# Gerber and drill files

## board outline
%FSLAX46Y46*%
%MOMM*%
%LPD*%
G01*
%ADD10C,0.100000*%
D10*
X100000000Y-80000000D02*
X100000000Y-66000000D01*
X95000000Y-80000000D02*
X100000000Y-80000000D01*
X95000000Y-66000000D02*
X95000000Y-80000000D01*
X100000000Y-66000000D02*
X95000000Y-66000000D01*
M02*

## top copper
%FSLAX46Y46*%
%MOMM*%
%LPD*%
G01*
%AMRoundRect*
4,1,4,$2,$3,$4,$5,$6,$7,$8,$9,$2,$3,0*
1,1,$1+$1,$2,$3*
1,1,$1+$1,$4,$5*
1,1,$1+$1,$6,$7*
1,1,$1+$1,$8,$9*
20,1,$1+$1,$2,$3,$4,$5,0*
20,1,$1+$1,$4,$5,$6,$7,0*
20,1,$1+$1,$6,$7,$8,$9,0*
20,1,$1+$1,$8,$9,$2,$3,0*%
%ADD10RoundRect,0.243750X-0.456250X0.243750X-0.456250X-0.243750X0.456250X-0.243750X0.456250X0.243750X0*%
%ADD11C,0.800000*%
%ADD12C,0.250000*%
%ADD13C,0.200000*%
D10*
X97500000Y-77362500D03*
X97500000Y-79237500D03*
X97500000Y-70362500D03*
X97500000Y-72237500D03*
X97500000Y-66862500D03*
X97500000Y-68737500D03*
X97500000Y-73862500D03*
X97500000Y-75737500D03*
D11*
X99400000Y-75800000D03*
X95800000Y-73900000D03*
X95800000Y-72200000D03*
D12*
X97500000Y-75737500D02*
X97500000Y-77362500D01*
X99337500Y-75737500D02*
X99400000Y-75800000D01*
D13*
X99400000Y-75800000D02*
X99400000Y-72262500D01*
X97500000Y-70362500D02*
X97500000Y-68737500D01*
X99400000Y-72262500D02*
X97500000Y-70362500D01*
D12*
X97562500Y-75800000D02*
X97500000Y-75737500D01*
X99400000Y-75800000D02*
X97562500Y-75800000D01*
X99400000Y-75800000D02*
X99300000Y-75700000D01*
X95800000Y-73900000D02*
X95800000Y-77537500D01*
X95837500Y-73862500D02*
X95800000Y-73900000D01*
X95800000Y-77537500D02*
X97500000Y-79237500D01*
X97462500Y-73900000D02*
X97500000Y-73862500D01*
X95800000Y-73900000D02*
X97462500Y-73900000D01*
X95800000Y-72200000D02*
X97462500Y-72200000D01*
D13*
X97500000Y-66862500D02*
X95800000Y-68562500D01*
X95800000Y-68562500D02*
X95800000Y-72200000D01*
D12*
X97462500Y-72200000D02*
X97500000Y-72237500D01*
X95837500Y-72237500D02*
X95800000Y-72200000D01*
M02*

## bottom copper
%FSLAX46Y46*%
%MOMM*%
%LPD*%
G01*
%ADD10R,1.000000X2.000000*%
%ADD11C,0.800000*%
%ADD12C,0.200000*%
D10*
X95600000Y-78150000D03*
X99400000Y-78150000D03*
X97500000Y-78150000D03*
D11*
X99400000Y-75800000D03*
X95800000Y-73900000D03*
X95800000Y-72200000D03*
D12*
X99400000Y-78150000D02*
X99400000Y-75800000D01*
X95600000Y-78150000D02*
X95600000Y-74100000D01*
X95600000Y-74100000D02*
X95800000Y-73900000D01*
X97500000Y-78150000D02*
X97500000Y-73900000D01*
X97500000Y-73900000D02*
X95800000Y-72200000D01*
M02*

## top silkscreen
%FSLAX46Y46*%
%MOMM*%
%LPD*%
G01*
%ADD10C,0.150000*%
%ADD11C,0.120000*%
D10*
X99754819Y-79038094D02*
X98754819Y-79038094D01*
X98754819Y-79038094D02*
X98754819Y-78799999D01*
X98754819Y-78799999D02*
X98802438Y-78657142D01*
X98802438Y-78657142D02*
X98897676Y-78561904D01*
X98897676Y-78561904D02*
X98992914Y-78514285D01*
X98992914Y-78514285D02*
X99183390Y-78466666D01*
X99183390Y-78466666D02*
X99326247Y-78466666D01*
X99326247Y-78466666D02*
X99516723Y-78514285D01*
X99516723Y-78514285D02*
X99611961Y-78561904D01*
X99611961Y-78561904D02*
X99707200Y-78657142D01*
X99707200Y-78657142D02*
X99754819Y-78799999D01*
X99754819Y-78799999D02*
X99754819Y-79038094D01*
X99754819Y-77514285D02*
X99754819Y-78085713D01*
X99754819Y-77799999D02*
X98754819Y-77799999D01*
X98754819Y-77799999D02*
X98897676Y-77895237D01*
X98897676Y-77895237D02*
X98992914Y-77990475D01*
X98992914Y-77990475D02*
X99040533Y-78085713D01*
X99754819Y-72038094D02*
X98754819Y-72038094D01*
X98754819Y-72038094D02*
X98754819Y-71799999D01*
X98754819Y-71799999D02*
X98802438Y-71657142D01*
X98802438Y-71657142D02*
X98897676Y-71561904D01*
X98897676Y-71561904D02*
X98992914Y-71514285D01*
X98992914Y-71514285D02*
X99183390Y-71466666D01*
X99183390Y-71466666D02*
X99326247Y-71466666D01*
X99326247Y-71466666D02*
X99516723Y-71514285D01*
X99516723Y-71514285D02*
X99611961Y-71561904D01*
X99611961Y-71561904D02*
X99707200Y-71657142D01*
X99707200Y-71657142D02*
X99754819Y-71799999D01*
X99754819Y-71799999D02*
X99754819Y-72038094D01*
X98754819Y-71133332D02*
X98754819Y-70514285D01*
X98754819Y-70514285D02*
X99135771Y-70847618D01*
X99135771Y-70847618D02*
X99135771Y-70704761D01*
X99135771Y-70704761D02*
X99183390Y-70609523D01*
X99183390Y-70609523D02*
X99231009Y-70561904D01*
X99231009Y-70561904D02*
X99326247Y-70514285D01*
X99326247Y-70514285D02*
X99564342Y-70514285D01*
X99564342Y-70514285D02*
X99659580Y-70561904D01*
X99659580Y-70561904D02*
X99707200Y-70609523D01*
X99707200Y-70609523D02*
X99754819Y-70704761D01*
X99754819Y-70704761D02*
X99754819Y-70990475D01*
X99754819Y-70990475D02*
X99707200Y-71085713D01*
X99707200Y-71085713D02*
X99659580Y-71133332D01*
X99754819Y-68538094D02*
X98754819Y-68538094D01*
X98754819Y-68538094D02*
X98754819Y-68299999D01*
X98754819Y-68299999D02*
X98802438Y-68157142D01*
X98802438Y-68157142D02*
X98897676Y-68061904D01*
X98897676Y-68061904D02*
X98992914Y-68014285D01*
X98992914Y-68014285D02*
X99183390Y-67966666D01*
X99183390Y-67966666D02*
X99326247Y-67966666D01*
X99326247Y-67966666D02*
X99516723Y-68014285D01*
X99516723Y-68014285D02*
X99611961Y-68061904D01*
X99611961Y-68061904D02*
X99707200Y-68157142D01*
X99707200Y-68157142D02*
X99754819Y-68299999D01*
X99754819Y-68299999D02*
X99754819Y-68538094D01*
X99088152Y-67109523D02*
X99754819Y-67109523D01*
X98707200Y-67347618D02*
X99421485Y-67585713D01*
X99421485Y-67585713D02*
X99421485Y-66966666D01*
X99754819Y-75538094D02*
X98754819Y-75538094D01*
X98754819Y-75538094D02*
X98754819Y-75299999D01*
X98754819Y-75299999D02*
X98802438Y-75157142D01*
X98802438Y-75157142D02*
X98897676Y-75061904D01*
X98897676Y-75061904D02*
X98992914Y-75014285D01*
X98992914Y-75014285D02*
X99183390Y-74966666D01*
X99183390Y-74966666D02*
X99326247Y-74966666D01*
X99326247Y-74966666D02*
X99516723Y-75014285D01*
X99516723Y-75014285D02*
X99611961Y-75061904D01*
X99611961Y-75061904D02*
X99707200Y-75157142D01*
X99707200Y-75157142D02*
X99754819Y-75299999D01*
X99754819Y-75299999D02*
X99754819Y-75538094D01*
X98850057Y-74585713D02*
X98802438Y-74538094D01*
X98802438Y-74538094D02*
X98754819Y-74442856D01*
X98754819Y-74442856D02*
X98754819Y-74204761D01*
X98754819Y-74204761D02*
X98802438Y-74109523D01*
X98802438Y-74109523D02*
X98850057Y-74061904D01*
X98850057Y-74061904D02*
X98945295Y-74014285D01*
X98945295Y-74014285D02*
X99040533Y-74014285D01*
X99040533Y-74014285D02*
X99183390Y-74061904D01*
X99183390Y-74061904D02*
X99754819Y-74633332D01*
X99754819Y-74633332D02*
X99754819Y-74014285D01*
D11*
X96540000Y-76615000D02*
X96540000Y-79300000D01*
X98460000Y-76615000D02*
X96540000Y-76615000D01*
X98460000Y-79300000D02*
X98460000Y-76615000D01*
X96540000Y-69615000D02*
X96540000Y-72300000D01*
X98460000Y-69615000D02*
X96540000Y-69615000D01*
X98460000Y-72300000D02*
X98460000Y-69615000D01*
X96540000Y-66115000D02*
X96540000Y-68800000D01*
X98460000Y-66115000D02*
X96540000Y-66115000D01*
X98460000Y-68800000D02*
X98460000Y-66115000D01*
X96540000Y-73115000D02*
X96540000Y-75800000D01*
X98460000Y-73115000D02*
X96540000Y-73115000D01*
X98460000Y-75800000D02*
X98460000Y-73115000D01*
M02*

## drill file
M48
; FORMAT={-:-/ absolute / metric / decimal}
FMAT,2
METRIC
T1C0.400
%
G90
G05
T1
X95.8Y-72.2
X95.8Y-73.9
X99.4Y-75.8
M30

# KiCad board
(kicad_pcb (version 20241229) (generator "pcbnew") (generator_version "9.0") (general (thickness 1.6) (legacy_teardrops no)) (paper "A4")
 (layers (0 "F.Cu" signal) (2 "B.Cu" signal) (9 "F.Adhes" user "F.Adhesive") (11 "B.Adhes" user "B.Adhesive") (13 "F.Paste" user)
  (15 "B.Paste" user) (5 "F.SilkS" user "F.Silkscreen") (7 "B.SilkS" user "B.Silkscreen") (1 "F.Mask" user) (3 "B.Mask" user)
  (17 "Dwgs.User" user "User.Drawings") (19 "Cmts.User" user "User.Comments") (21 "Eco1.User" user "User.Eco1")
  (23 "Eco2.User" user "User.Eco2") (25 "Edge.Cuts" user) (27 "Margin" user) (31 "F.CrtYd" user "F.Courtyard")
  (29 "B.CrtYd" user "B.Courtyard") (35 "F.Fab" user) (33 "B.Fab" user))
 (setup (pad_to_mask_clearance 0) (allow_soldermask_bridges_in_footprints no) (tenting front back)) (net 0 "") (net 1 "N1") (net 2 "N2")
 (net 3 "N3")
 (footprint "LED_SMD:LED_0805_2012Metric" (layer "F.Cu") (at 97.5 78.3 -90)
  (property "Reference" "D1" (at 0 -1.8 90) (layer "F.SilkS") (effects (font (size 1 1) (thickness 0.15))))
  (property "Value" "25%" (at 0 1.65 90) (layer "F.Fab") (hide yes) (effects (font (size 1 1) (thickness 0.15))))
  (fp_line (start -1.685 0.96) (end 1 0.96) (stroke (width 0.12) (type solid)) (layer "F.SilkS"))
  (fp_line (start -1.685 -0.96) (end -1.685 0.96) (stroke (width 0.12) (type solid)) (layer "F.SilkS"))
  (fp_line (start 1 -0.96) (end -1.685 -0.96) (stroke (width 0.12) (type solid)) (layer "F.SilkS"))
  (pad "1" smd roundrect (at -0.9375 0 270) (size 0.975 1.4) (layers "F.Cu" "F.Mask" "F.Paste") (roundrect_rratio 0.25) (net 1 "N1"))
  (pad "2" smd roundrect (at 0.9375 0 270) (size 0.975 1.4) (layers "F.Cu" "F.Mask" "F.Paste") (roundrect_rratio 0.25) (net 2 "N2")))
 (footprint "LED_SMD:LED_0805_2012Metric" (layer "F.Cu") (at 97.5 71.3 -90)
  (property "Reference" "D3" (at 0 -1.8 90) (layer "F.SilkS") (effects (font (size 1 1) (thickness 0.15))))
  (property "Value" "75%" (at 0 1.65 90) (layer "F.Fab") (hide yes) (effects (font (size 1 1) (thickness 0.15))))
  (fp_line (start -1.685 0.96) (end 1 0.96) (stroke (width 0.12) (type solid)) (layer "F.SilkS"))
  (fp_line (start -1.685 -0.96) (end -1.685 0.96) (stroke (width 0.12) (type solid)) (layer "F.SilkS"))
  (fp_line (start 1 -0.96) (end -1.685 -0.96) (stroke (width 0.12) (type solid)) (layer "F.SilkS"))
  (pad "1" smd roundrect (at -0.9375 0 270) (size 0.975 1.4) (layers "F.Cu" "F.Mask" "F.Paste") (roundrect_rratio 0.25) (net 1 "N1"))
  (pad "2" smd roundrect (at 0.9375 0 270) (size 0.975 1.4) (layers "F.Cu" "F.Mask" "F.Paste") (roundrect_rratio 0.25) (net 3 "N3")))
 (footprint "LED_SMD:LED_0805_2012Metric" (layer "F.Cu") (at 97.5 67.8 -90)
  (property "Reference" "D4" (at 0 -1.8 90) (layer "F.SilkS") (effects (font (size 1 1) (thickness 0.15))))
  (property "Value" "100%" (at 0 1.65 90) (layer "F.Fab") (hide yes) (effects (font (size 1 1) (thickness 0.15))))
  (fp_line (start -1.685 0.96) (end 1 0.96) (stroke (width 0.12) (type solid)) (layer "F.SilkS"))
  (fp_line (start -1.685 -0.96) (end -1.685 0.96) (stroke (width 0.12) (type solid)) (layer "F.SilkS"))
  (fp_line (start 1 -0.96) (end -1.685 -0.96) (stroke (width 0.12) (type solid)) (layer "F.SilkS"))
  (pad "1" smd roundrect (at -0.9375 0 270) (size 0.975 1.4) (layers "F.Cu" "F.Mask" "F.Paste") (roundrect_rratio 0.25) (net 3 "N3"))
  (pad "2" smd roundrect (at 0.9375 0 270) (size 0.975 1.4) (layers "F.Cu" "F.Mask" "F.Paste") (roundrect_rratio 0.25) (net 1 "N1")))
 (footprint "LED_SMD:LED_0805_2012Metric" (layer "F.Cu") (at 97.5 74.8 -90)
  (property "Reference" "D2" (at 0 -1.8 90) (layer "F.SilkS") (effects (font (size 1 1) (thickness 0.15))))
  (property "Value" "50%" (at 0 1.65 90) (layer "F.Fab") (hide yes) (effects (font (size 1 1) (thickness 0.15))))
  (fp_line (start -1.685 0.96) (end 1 0.96) (stroke (width 0.12) (type solid)) (layer "F.SilkS"))
  (fp_line (start -1.685 -0.96) (end -1.685 0.96) (stroke (width 0.12) (type solid)) (layer "F.SilkS"))
  (fp_line (start 1 -0.96) (end -1.685 -0.96) (stroke (width 0.12) (type solid)) (layer "F.SilkS"))
  (pad "1" smd roundrect (at -0.9375 0 270) (size 0.975 1.4) (layers "F.Cu" "F.Mask" "F.Paste") (roundrect_rratio 0.25) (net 2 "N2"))
  (pad "2" smd roundrect (at 0.9375 0 270) (size 0.975 1.4) (layers "F.Cu" "F.Mask" "F.Paste") (roundrect_rratio 0.25) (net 1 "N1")))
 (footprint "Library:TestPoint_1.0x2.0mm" (layer "B.Cu") (at 95.6 78.15 180)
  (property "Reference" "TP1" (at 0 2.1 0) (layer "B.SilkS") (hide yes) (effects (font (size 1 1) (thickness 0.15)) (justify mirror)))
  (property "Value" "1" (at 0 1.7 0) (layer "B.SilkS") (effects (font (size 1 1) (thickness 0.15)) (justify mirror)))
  (pad "1" smd rect (at 0 0 180) (size 1 2) (layers "B.Cu" "B.Mask") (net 2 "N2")))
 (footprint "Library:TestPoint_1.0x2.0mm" (layer "B.Cu") (at 99.4 78.15 180)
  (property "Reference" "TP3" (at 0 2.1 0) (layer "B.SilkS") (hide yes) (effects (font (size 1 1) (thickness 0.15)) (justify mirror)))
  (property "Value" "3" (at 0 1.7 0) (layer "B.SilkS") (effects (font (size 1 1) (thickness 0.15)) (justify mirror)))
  (pad "3" smd rect (at 0 0 180) (size 1 2) (layers "B.Cu" "B.Mask") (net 1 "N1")))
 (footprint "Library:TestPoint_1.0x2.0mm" (layer "B.Cu") (at 97.5 78.15 180)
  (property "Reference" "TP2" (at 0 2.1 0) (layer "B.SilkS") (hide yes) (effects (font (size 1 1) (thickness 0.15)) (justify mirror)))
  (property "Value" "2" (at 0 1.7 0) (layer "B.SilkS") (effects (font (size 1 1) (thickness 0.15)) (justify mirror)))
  (pad "2" smd rect (at 0 0 180) (size 1 2) (layers "B.Cu" "B.Mask") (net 3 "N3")))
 (gr_line (start 100 80) (end 100 66) (stroke (width 0.1) (type solid)) (layer "Edge.Cuts"))
 (gr_line (start 95 80) (end 100 80) (stroke (width 0.1) (type solid)) (layer "Edge.Cuts"))
 (gr_line (start 95 66) (end 95 80) (stroke (width 0.1) (type solid)) (layer "Edge.Cuts"))
 (gr_line (start 100 66) (end 95 66) (stroke (width 0.1) (type solid)) (layer "Edge.Cuts"))
 (segment (start 97.5 75.7375) (end 97.5 77.3625) (width 0.25) (layer "F.Cu") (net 1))
 (segment (start 99.3375 75.7375) (end 99.4 75.8) (width 0.25) (layer "F.Cu") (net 1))
 (segment (start 99.4 75.8) (end 99.4 72.2625) (width 0.2) (layer "F.Cu") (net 1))
 (segment (start 97.5 70.3625) (end 97.5 68.7375) (width 0.2) (layer "F.Cu") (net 1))
 (segment (start 99.4 72.2625) (end 97.5 70.3625) (width 0.2) (layer "F.Cu") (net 1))
 (segment (start 97.5625 75.8) (end 97.5 75.7375) (width 0.25) (layer "F.Cu") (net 1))
 (segment (start 99.4 75.8) (end 97.5625 75.8) (width 0.25) (layer "F.Cu") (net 1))
 (segment (start 99.4 75.8) (end 99.3 75.7) (width 0.25) (layer "F.Cu") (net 1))
 (via (at 99.4 75.8) (size 0.8) (drill 0.4) (layers "F.Cu" "B.Cu") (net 1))
 (segment (start 99.4 78.15) (end 99.4 75.8) (width 0.2) (layer "B.Cu") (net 1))
 (segment (start 95.8 73.9) (end 95.8 77.5375) (width 0.25) (layer "F.Cu") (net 2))
 (segment (start 95.8375 73.8625) (end 95.8 73.9) (width 0.25) (layer "F.Cu") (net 2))
 (segment (start 95.8 77.5375) (end 97.5 79.2375) (width 0.25) (layer "F.Cu") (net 2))
 (segment (start 97.4625 73.9) (end 97.5 73.8625) (width 0.25) (layer "F.Cu") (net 2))
 (segment (start 95.8 73.9) (end 97.4625 73.9) (width 0.25) (layer "F.Cu") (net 2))
 (via (at 95.8 73.9) (size 0.8) (drill 0.4) (layers "F.Cu" "B.Cu") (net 2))
 (segment (start 95.6 78.15) (end 95.6 74.1) (width 0.2) (layer "B.Cu") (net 2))
 (segment (start 95.6 74.1) (end 95.8 73.9) (width 0.2) (layer "B.Cu") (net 2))
 (segment (start 95.8 72.2) (end 97.4625 72.2) (width 0.25) (layer "F.Cu") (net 3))
 (segment (start 97.5 66.8625) (end 95.8 68.5625) (width 0.2) (layer "F.Cu") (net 3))
 (segment (start 95.8 68.5625) (end 95.8 72.2) (width 0.2) (layer "F.Cu") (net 3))
 (segment (start 97.4625 72.2) (end 97.5 72.2375) (width 0.25) (layer "F.Cu") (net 3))
 (segment (start 95.8375 72.2375) (end 95.8 72.2) (width 0.25) (layer "F.Cu") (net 3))
 (via (at 95.8 72.2) (size 0.8) (drill 0.4) (layers "F.Cu" "B.Cu") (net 3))
 (segment (start 97.5 78.15) (end 97.5 73.9) (width 0.2) (layer "B.Cu") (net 3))
 (segment (start 97.5 73.9) (end 95.8 72.2) (width 0.2) (layer "B.Cu") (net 3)))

